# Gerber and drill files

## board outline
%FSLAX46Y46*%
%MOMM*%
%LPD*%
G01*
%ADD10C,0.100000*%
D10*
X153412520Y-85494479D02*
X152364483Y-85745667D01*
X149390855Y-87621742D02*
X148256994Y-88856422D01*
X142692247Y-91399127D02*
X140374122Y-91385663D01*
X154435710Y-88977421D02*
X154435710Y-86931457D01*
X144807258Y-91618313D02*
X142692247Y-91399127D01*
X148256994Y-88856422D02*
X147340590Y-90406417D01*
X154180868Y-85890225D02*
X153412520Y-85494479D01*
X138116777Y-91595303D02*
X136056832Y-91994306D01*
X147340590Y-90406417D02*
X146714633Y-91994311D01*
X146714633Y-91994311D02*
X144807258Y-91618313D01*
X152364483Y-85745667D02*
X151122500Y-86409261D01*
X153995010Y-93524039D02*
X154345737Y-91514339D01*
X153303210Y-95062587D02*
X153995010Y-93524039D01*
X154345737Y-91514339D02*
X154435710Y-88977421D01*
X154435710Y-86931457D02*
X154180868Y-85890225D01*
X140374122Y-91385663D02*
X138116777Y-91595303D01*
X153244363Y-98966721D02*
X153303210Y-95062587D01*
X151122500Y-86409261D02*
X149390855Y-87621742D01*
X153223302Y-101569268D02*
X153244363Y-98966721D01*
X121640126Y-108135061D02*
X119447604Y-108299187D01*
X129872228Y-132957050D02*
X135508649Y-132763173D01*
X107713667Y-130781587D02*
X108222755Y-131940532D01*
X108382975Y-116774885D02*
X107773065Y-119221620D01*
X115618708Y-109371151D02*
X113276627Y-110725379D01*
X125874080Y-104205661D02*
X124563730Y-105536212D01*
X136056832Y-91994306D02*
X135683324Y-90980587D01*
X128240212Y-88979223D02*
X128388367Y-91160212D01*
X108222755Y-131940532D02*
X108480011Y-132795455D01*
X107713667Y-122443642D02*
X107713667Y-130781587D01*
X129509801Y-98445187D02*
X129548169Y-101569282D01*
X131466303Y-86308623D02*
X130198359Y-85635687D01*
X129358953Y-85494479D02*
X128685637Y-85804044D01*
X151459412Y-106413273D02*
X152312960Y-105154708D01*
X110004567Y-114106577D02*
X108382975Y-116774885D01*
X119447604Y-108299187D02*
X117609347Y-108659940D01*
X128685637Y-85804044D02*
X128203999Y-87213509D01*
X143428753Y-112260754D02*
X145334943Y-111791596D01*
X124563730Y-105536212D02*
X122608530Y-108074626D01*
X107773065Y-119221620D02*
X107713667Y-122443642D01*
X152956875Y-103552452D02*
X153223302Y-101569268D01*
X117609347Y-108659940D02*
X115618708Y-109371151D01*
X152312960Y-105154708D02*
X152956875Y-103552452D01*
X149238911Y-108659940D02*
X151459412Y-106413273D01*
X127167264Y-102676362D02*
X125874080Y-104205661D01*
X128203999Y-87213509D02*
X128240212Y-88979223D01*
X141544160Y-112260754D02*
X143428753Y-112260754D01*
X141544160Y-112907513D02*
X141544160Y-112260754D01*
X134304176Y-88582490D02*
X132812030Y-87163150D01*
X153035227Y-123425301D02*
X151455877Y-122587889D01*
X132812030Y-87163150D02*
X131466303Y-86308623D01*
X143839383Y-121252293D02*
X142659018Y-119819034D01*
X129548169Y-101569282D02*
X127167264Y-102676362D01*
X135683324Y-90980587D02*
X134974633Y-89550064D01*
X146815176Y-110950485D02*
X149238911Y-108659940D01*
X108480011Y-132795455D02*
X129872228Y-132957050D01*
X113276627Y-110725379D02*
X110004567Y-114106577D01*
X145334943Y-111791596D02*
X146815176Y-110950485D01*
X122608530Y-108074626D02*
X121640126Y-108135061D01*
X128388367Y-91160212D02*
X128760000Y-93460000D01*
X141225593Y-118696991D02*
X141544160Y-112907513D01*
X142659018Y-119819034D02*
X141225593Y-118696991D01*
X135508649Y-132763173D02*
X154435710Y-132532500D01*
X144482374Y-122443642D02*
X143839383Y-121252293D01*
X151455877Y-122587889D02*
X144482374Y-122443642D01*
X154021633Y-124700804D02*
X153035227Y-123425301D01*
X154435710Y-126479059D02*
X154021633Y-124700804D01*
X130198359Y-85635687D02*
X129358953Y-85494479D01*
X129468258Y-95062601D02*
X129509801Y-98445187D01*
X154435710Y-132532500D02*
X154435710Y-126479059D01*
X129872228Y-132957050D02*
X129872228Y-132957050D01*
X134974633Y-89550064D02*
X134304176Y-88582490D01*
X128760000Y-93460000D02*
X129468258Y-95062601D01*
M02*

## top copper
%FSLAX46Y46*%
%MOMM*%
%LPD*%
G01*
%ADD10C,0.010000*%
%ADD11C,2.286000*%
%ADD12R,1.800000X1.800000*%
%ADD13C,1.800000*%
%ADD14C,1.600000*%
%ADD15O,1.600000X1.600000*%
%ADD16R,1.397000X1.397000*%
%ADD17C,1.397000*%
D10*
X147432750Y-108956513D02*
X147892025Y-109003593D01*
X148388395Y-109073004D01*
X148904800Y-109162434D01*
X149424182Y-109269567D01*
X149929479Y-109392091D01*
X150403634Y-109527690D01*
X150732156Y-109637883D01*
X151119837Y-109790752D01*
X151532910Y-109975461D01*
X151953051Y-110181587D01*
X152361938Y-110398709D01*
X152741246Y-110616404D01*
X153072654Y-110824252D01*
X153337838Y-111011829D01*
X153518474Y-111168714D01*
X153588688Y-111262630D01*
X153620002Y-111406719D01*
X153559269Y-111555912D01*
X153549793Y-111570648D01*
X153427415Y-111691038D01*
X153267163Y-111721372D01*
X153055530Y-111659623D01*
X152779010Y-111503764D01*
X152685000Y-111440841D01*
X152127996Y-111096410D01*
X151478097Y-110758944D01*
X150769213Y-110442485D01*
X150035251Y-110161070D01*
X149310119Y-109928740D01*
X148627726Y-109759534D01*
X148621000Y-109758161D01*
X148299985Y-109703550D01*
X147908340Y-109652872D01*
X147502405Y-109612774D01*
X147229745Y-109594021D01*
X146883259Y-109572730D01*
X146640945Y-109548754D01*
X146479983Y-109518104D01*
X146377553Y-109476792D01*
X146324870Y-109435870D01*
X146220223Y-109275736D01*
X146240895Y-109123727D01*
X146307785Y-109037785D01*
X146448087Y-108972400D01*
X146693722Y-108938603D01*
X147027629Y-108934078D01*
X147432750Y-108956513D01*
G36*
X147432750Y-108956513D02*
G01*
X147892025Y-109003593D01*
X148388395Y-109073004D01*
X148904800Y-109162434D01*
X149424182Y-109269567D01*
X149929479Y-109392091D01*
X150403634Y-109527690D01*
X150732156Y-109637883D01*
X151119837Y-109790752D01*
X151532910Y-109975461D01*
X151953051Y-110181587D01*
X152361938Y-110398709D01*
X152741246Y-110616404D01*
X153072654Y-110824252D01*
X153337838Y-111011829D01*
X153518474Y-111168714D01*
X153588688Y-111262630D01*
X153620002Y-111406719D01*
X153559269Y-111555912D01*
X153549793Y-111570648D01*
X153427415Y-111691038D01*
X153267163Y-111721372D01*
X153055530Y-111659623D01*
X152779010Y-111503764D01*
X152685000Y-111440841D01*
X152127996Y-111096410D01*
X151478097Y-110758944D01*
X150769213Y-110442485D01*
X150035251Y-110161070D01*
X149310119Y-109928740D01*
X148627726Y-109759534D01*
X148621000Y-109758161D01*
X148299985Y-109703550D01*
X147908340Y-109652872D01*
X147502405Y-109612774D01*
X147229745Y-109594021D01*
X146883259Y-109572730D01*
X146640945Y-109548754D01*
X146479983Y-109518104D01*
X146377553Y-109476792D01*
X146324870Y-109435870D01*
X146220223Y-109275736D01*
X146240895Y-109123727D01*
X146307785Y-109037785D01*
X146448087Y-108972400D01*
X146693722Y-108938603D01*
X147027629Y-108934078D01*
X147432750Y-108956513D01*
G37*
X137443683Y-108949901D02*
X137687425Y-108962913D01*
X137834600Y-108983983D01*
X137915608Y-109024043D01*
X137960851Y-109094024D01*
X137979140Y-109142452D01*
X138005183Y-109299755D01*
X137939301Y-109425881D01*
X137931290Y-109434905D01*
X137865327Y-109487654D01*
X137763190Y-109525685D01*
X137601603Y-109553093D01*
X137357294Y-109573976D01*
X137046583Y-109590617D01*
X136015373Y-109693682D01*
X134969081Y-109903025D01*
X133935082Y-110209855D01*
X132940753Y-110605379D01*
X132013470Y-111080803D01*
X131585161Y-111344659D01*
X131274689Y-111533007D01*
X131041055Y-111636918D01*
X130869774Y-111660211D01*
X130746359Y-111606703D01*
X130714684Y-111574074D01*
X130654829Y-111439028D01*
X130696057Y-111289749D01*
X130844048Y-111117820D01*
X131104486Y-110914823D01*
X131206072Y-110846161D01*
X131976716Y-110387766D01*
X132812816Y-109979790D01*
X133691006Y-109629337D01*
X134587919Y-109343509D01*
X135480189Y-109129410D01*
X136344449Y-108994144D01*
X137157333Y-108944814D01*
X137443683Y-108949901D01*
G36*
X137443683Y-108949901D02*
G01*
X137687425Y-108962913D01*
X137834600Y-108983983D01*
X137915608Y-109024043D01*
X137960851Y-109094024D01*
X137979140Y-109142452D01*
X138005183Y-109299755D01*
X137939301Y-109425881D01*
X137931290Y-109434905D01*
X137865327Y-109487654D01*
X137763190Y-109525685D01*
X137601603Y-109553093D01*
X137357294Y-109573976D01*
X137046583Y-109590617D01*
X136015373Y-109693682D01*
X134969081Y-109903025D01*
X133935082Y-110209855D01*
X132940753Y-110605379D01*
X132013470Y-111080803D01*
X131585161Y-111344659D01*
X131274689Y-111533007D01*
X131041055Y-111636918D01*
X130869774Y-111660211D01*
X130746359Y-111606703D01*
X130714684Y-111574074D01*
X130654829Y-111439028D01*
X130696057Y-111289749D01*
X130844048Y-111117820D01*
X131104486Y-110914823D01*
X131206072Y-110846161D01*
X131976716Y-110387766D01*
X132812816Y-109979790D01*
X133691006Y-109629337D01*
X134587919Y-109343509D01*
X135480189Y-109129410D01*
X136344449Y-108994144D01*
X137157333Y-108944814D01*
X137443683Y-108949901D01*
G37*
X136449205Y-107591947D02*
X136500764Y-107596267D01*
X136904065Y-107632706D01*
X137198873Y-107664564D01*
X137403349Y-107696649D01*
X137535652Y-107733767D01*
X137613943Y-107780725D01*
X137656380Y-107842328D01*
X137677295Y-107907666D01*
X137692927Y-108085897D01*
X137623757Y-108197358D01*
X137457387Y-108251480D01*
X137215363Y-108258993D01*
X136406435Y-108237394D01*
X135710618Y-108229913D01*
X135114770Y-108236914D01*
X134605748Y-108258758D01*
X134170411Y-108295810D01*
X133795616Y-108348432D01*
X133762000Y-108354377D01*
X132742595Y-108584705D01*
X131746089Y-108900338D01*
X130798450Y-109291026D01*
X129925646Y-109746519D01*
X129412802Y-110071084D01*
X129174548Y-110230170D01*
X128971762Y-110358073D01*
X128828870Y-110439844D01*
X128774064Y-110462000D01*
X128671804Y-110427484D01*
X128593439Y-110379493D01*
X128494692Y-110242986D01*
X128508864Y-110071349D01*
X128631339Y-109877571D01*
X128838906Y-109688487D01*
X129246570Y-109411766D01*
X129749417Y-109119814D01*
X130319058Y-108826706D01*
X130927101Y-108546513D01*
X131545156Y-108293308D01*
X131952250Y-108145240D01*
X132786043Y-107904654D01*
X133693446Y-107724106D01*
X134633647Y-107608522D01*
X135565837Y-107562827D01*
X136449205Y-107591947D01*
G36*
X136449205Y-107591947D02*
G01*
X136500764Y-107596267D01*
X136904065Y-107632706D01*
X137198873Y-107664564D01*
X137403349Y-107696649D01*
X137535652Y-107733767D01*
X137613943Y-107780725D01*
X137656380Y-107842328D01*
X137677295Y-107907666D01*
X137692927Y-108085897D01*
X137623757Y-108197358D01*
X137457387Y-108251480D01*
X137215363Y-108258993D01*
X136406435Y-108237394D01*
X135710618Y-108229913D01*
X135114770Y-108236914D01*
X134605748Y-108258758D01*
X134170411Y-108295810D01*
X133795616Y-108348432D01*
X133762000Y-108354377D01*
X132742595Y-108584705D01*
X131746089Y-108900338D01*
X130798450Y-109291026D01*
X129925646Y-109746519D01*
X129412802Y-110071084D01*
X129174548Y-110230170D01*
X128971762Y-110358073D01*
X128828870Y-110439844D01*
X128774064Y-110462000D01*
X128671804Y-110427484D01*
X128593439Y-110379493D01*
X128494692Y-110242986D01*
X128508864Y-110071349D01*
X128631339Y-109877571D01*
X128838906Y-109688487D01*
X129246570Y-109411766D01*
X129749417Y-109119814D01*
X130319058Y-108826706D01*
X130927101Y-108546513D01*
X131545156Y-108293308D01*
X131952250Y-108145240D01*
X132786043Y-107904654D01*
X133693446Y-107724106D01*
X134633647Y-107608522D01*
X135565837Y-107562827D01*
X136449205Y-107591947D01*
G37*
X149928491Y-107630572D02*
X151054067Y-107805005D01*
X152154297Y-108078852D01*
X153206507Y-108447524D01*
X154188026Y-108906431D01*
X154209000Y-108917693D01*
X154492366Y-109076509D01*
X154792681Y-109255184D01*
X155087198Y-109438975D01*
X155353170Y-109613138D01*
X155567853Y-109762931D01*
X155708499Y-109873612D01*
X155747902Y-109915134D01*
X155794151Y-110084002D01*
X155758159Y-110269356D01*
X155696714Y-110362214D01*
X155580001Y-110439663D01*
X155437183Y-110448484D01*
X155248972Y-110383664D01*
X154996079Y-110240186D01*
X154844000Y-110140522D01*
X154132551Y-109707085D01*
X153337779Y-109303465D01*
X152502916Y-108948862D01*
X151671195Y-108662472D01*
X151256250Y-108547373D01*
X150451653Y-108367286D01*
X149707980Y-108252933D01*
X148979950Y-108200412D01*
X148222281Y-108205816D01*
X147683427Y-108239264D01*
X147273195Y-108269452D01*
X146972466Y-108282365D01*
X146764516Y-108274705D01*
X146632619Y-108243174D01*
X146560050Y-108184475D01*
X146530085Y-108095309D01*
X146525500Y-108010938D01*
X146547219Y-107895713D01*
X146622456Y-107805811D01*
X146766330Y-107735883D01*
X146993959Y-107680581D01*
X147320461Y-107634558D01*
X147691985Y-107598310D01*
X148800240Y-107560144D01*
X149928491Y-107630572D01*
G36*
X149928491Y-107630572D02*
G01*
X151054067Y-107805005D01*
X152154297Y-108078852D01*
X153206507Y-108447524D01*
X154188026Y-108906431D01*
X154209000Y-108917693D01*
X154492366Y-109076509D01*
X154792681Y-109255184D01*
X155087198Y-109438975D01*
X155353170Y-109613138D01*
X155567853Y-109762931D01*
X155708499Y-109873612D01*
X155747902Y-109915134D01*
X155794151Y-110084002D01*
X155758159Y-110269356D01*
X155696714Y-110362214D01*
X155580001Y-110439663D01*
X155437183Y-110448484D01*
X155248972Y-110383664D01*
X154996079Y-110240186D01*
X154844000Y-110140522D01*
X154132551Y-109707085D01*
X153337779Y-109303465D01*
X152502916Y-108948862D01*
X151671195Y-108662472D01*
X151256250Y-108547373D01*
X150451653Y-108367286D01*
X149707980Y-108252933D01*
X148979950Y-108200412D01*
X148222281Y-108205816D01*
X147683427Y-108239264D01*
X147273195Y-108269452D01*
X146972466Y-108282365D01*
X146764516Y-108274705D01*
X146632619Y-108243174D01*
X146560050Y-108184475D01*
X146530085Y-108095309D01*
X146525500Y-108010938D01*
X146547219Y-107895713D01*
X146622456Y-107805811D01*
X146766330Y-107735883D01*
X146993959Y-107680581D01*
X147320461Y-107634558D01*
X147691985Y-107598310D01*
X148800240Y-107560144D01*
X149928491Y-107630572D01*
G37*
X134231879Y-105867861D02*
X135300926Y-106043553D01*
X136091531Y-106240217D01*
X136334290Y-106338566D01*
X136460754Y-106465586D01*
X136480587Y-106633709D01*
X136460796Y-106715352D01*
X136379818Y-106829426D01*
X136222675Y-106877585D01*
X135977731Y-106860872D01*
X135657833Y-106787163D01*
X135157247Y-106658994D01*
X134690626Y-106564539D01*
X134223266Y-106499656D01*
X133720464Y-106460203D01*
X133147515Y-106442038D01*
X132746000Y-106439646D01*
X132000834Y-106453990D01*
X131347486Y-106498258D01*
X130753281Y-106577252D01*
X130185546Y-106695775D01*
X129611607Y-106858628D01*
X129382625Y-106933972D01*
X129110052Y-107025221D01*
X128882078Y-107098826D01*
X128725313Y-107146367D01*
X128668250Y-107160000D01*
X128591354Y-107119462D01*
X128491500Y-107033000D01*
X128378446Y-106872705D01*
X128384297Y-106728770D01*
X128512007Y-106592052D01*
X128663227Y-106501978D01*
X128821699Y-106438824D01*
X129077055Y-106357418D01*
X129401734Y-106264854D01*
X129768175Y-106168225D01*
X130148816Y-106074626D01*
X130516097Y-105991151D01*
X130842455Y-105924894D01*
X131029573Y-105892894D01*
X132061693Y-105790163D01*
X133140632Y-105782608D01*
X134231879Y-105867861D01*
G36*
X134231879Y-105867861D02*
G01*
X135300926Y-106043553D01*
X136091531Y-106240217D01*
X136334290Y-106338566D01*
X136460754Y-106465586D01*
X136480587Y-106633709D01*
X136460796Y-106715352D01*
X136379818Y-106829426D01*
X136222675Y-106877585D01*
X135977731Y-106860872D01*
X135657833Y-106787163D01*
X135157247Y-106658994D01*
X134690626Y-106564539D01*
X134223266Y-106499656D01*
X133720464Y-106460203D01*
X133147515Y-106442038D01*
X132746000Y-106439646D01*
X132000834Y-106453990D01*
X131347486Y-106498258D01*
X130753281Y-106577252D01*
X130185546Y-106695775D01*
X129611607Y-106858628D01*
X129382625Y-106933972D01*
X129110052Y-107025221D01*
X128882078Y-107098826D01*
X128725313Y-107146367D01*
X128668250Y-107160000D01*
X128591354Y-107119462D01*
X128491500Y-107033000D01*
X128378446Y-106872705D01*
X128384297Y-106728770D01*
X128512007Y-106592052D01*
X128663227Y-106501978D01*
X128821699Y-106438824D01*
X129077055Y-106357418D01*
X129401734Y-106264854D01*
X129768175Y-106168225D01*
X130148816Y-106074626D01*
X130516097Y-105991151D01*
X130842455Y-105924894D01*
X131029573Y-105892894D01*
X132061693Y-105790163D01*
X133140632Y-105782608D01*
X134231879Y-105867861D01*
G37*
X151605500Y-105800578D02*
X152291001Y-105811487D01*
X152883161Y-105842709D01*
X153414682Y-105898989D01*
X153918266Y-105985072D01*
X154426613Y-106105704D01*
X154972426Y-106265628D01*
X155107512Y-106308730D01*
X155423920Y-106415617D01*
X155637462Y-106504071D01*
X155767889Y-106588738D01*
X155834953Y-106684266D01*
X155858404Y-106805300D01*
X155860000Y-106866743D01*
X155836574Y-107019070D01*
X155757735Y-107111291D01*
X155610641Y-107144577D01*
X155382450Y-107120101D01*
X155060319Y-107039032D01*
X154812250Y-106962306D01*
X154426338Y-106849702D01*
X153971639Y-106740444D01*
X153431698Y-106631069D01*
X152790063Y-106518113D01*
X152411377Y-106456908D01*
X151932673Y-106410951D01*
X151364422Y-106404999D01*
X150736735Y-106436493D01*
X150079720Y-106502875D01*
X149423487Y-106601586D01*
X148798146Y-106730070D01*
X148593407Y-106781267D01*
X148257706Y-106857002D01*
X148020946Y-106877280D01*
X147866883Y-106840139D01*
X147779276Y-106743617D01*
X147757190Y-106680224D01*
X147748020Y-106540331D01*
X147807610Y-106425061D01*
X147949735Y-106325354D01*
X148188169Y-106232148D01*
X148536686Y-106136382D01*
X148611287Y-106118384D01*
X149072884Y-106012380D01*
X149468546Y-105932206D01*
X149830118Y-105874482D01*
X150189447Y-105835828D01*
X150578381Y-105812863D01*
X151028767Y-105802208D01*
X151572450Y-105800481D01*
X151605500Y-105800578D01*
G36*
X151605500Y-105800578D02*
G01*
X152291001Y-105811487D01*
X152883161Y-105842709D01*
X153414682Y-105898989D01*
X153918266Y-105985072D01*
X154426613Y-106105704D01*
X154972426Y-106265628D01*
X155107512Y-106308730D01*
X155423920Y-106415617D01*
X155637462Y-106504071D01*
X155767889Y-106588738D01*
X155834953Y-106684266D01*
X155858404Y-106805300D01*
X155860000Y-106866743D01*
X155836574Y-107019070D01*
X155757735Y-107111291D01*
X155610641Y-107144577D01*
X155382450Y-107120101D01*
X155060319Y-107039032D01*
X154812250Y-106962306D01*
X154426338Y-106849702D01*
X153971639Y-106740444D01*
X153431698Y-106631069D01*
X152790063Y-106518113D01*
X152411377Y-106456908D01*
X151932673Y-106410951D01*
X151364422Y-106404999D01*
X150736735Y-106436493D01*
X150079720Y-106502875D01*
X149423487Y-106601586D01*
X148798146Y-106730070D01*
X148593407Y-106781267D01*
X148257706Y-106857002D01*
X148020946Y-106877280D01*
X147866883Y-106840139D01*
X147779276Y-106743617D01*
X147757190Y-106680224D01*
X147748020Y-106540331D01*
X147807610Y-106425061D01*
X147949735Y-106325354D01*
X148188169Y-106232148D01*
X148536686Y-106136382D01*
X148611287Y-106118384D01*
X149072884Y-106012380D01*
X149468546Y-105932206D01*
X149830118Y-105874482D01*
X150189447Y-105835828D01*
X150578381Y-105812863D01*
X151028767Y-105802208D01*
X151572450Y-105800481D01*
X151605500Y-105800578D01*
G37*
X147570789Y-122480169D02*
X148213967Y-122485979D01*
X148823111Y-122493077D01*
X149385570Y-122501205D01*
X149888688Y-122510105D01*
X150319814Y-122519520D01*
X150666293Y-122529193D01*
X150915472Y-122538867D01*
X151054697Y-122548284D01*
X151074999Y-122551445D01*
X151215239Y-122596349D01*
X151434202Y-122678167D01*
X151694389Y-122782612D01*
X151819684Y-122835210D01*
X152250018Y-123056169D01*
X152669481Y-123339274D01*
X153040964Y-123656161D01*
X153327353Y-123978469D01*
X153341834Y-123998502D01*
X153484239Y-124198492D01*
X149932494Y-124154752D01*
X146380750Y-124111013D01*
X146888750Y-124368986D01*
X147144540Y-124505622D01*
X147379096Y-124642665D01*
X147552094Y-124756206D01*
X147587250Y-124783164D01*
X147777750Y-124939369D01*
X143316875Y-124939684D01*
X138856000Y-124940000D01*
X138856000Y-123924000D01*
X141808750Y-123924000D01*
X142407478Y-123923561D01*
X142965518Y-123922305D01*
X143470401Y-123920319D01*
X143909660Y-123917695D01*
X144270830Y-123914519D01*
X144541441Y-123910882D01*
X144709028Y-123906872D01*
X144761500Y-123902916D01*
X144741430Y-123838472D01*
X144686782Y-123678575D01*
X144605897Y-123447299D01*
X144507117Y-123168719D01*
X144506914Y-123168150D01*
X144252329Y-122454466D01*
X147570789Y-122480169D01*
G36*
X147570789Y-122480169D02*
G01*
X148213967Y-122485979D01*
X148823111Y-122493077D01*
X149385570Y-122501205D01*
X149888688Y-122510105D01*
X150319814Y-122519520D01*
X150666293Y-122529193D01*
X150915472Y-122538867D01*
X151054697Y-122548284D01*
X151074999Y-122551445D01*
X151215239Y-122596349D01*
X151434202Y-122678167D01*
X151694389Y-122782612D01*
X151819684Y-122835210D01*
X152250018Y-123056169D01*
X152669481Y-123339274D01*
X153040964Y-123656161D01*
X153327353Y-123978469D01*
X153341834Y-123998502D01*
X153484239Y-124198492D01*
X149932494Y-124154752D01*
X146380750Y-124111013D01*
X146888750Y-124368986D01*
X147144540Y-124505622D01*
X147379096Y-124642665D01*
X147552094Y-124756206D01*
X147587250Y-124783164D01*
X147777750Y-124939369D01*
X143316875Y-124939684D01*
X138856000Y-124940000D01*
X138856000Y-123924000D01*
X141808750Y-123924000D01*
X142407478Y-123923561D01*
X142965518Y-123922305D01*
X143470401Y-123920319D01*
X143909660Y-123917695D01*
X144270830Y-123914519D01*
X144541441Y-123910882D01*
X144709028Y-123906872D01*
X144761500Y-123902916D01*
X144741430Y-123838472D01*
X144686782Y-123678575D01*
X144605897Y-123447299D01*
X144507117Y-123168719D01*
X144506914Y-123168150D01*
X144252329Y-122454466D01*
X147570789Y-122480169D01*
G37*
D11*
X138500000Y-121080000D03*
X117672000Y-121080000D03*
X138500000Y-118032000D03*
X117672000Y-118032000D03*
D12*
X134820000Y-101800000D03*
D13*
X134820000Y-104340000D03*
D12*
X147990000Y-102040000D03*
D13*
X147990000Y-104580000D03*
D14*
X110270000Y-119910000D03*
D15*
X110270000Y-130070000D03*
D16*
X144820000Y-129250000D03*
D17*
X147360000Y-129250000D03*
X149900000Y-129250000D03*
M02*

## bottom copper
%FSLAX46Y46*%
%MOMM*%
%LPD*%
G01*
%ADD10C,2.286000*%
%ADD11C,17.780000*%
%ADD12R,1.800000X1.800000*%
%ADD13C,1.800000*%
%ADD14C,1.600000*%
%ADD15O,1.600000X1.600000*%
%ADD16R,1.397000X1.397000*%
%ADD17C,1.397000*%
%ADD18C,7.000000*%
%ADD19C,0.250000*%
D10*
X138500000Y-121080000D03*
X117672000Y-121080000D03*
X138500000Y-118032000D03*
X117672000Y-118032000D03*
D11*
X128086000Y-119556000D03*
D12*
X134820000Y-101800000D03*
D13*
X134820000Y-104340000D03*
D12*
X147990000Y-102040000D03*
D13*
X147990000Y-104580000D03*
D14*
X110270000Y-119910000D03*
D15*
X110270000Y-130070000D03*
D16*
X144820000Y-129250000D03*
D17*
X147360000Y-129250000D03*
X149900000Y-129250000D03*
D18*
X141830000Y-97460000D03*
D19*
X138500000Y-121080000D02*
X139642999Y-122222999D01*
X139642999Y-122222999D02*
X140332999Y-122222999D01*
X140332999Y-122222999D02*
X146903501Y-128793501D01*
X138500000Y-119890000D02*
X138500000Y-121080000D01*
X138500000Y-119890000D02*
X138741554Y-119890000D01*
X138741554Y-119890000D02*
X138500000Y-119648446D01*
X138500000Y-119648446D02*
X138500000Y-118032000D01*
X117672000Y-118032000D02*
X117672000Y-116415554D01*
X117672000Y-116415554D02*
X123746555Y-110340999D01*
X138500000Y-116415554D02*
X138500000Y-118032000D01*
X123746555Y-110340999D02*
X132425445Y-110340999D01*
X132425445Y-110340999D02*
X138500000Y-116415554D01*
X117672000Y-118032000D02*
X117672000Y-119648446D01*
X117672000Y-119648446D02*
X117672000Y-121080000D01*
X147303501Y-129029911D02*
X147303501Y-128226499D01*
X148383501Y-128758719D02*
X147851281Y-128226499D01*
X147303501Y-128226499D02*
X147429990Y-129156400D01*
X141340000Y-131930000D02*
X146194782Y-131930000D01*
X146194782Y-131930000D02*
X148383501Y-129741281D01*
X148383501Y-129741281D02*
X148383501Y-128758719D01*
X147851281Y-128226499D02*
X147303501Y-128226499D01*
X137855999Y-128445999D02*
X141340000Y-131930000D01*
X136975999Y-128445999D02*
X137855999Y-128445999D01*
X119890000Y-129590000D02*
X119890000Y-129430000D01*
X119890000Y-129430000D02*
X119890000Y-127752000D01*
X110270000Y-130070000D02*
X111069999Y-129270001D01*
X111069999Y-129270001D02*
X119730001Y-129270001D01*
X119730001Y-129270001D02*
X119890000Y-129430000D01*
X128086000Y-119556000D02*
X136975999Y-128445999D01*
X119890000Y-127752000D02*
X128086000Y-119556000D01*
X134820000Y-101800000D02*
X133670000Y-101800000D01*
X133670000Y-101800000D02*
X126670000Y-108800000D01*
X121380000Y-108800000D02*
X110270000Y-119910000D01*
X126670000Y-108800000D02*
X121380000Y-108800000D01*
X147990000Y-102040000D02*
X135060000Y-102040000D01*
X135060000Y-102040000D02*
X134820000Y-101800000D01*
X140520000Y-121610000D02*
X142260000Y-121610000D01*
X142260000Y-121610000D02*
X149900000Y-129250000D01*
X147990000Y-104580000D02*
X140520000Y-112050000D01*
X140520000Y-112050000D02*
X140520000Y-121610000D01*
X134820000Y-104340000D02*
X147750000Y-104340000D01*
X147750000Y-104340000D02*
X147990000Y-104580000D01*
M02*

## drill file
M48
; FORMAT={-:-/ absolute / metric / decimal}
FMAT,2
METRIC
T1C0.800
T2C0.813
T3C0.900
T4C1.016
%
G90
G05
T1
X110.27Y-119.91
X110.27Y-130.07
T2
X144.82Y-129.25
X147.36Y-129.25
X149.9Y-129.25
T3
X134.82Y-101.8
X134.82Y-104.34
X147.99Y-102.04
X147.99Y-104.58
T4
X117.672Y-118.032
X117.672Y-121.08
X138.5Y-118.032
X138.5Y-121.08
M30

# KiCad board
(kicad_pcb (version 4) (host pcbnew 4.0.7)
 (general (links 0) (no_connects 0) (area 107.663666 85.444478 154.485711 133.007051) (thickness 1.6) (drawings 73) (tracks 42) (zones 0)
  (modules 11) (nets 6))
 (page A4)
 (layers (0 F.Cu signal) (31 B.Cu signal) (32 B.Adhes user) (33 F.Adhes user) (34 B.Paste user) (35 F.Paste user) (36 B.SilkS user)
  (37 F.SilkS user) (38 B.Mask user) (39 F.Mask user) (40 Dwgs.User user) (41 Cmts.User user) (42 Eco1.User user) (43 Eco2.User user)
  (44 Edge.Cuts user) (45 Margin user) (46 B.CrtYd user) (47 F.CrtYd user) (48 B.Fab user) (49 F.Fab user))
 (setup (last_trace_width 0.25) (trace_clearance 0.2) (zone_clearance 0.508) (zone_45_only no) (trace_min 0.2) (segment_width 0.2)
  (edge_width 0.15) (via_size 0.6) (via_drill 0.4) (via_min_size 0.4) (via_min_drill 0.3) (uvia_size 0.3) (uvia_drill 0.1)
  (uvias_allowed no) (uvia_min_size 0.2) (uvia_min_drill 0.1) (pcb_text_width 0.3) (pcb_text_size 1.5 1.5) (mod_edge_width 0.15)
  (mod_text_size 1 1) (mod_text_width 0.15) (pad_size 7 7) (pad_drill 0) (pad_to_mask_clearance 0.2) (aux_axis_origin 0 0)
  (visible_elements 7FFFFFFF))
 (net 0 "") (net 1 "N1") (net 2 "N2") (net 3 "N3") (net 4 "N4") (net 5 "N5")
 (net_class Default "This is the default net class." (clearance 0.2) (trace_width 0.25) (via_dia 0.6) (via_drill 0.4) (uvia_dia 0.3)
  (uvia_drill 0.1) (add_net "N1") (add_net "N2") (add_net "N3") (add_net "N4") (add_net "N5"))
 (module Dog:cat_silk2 (layer F.Cu) (at 130.76 109.63)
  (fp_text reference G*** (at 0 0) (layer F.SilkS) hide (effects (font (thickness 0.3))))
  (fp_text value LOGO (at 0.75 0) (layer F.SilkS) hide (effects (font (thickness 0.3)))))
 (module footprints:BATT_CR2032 (layer B.Cu) (at 128.086 119.556 180)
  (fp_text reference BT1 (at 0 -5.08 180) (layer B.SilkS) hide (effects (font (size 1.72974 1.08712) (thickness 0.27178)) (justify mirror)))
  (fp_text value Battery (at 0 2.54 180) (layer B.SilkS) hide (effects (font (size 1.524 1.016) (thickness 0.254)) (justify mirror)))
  (pad 1 thru_hole circle (at -10.414 -1.524 180) (size 2.286 2.286) (drill 1.016) (layers *.Cu *.Mask B.SilkS) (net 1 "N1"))
  (pad 1 thru_hole circle (at 10.414 -1.524 180) (size 2.286 2.286) (drill 1.016) (layers *.Cu *.Mask B.SilkS) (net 1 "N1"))
  (pad 1 thru_hole circle (at -10.414 1.524 180) (size 2.286 2.286) (drill 1.016) (layers *.Cu *.Mask B.SilkS) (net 1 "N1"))
  (pad 1 thru_hole circle (at 10.414 1.524 180) (size 2.286 2.286) (drill 1.016) (layers *.Cu *.Mask B.SilkS) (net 1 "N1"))
  (pad 2 smd circle (at 0 0 180) (size 17.78 17.78) (layers B.Cu B.Paste B.Mask) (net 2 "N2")))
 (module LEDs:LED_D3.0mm (layer F.Cu) (at 134.82 101.8 270)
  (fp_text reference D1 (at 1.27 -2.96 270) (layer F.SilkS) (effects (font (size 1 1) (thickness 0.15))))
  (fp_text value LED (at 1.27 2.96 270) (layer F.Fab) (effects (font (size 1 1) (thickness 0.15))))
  (pad 1 thru_hole rect (at 0 0 270) (size 1.8 1.8) (drill 0.9) (layers *.Cu *.Mask) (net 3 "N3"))
  (pad 2 thru_hole circle (at 2.54 0 270) (size 1.8 1.8) (drill 0.9) (layers *.Cu *.Mask) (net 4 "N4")))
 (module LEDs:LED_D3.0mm (layer F.Cu) (at 147.99 102.04 270)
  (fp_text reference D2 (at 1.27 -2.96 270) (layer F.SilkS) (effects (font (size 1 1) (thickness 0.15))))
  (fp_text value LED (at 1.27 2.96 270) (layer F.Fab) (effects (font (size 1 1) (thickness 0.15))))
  (pad 1 thru_hole rect (at 0 0 270) (size 1.8 1.8) (drill 0.9) (layers *.Cu *.Mask) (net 3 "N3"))
  (pad 2 thru_hole circle (at 2.54 0 270) (size 1.8 1.8) (drill 0.9) (layers *.Cu *.Mask) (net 4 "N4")))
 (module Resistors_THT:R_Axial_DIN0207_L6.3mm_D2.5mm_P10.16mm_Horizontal (layer B.Cu) (at 110.27 119.91 270)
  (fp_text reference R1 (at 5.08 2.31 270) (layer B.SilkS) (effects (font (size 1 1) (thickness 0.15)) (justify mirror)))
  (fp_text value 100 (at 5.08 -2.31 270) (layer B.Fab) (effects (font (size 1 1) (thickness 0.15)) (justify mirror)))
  (pad 1 thru_hole circle (at 0 0 270) (size 1.6 1.6) (drill 0.8) (layers *.Cu *.Mask) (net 3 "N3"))
  (pad 2 thru_hole oval (at 10.16 0 270) (size 1.6 1.6) (drill 0.8) (layers *.Cu *.Mask) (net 2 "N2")))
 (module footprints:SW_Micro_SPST (layer B.Cu) (at 147.36 129.25)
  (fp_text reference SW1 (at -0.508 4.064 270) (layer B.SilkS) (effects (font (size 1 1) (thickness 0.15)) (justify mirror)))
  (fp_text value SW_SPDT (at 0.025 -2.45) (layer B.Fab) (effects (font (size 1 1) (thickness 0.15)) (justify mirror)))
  (pad 1 thru_hole rect (at -2.54 0) (size 1.397 1.397) (drill 0.8128) (layers *.Cu *.Mask B.SilkS) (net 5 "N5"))
  (pad 2 thru_hole circle (at 0 0) (size 1.397 1.397) (drill 0.8128) (layers *.Cu *.Mask B.SilkS) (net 1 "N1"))
  (pad 3 thru_hole circle (at 2.54 0) (size 1.397 1.397) (drill 0.8128) (layers *.Cu *.Mask B.SilkS) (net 4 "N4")))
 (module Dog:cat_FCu (layer F.Cu) (at 131.73 110.97)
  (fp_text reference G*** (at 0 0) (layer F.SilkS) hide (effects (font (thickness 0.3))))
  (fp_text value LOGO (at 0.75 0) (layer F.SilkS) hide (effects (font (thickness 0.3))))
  (fp_poly
   (pts (xy 15.70275 -2.013487) (xy 16.162025 -1.966407) (xy 16.658395 -1.896996) (xy 17.1748 -1.807566) (xy 17.694182 -1.700433)
    (xy 18.199479 -1.577909) (xy 18.673634 -1.44231) (xy 19.002156 -1.332117) (xy 19.389837 -1.179248) (xy 19.80291 -0.994539)
    (xy 20.223051 -0.788413) (xy 20.631938 -0.571291) (xy 21.011246 -0.353596) (xy 21.342654 -0.145748) (xy 21.607838 0.041829)
    (xy 21.788474 0.198714) (xy 21.858688 0.29263) (xy 21.890002 0.436719) (xy 21.829269 0.585912) (xy 21.819793 0.600648)
    (xy 21.697415 0.721038) (xy 21.537163 0.751372) (xy 21.32553 0.689623) (xy 21.04901 0.533764) (xy 20.955 0.470841)
    (xy 20.397996 0.12641) (xy 19.748097 -0.211056) (xy 19.039213 -0.527515) (xy 18.305251 -0.80893) (xy 17.580119 -1.04126)
    (xy 16.897726 -1.210466) (xy 16.891 -1.211839) (xy 16.569985 -1.26645) (xy 16.17834 -1.317128) (xy 15.772405 -1.357226)
    (xy 15.499745 -1.375979) (xy 15.153259 -1.39727) (xy 14.910945 -1.421246) (xy 14.749983 -1.451896) (xy 14.647553 -1.493208)
    (xy 14.59487 -1.53413) (xy 14.490223 -1.694264) (xy 14.510895 -1.846273) (xy 14.577785 -1.932215) (xy 14.718087 -1.9976)
    (xy 14.963722 -2.031397) (xy 15.297629 -2.035922) (xy 15.70275 -2.013487))
   (layer F.Cu) (width 0.01))
  (fp_poly
   (pts (xy 5.713683 -2.020099) (xy 5.957425 -2.007087) (xy 6.1046 -1.986017) (xy 6.185608 -1.945957) (xy 6.230851 -1.875976)
    (xy 6.24914 -1.827548) (xy 6.275183 -1.670245) (xy 6.209301 -1.544119) (xy 6.20129 -1.535095) (xy 6.135327 -1.482346)
    (xy 6.03319 -1.444315) (xy 5.871603 -1.416907) (xy 5.627294 -1.396024) (xy 5.316583 -1.379383) (xy 4.285373 -1.276318)
    (xy 3.239081 -1.066975) (xy 2.205082 -0.760145) (xy 1.210753 -0.364621) (xy 0.28347 0.110803) (xy -0.144839 0.374659)
    (xy -0.455311 0.563007) (xy -0.688945 0.666918) (xy -0.860226 0.690211) (xy -0.983641 0.636703) (xy -1.015316 0.604074)
    (xy -1.075171 0.469028) (xy -1.033943 0.319749) (xy -0.885952 0.14782) (xy -0.625514 -0.055177) (xy -0.523928 -0.123839)
    (xy 0.246716 -0.582234) (xy 1.082816 -0.99021) (xy 1.961006 -1.340663) (xy 2.857919 -1.626491) (xy 3.750189 -1.84059)
    (xy 4.614449 -1.975856) (xy 5.427333 -2.025186) (xy 5.713683 -2.020099))
   (layer F.Cu) (width 0.01))
  (fp_poly
   (pts (xy 4.719205 -3.378053) (xy 4.770764 -3.373733) (xy 5.174065 -3.337294) (xy 5.468873 -3.305436) (xy 5.673349 -3.273351)
    (xy 5.805652 -3.236233) (xy 5.883943 -3.189275) (xy 5.92638 -3.127672) (xy 5.947295 -3.062334) (xy 5.962927 -2.884103)
    (xy 5.893757 -2.772642) (xy 5.727387 -2.71852) (xy 5.485363 -2.711007) (xy 4.676435 -2.732606) (xy 3.980618 -2.740087)
    (xy 3.38477 -2.733086) (xy 2.875748 -2.711242) (xy 2.440411 -2.67419) (xy 2.065616 -2.621568) (xy 2.032 -2.615623)
    (xy 1.012595 -2.385295) (xy 0.016089 -2.069662) (xy -0.93155 -1.678974) (xy -1.804354 -1.223481) (xy -2.317198 -0.898916)
    (xy -2.555452 -0.73983) (xy -2.758238 -0.611927) (xy -2.90113 -0.530156) (xy -2.955936 -0.508) (xy -3.058196 -0.542516)
    (xy -3.136561 -0.590507) (xy -3.235308 -0.727014) (xy -3.221136 -0.898651) (xy -3.098661 -1.092429) (xy -2.891094 -1.281513)
    (xy -2.48343 -1.558234) (xy -1.980583 -1.850186) (xy -1.410942 -2.143294) (xy -0.802899 -2.423487) (xy -0.184844 -2.676692)
    (xy 0.22225 -2.82476) (xy 1.056043 -3.065346) (xy 1.963446 -3.245894) (xy 2.903647 -3.361478) (xy 3.835837 -3.407173)
    (xy 4.719205 -3.378053))
   (layer F.Cu) (width 0.01))
  (fp_poly
   (pts (xy 18.198491 -3.339428) (xy 19.324067 -3.164995) (xy 20.424297 -2.891148) (xy 21.476507 -2.522476) (xy 22.458026 -2.063569)
    (xy 22.479 -2.052307) (xy 22.762366 -1.893491) (xy 23.062681 -1.714816) (xy 23.357198 -1.531025) (xy 23.62317 -1.356862)
    (xy 23.837853 -1.207069) (xy 23.978499 -1.096388) (xy 24.017902 -1.054866) (xy 24.064151 -0.885998) (xy 24.028159 -0.700644)
    (xy 23.966714 -0.607786) (xy 23.850001 -0.530337) (xy 23.707183 -0.521516) (xy 23.518972 -0.586336) (xy 23.266079 -0.729814)
    (xy 23.114 -0.829478) (xy 22.402551 -1.262915) (xy 21.607779 -1.666535) (xy 20.772916 -2.021138) (xy 19.941195 -2.307528)
    (xy 19.52625 -2.422627) (xy 18.721653 -2.602714) (xy 17.97798 -2.717067) (xy 17.24995 -2.769588) (xy 16.492281 -2.764184)
    (xy 15.953427 -2.730736) (xy 15.543195 -2.700548) (xy 15.242466 -2.687635) (xy 15.034516 -2.695295) (xy 14.902619 -2.726826)
    (xy 14.83005 -2.785525) (xy 14.800085 -2.874691) (xy 14.7955 -2.959062) (xy 14.817219 -3.074287) (xy 14.892456 -3.164189)
    (xy 15.03633 -3.234117) (xy 15.263959 -3.289419) (xy 15.590461 -3.335442) (xy 15.961985 -3.37169) (xy 17.07024 -3.409856)
    (xy 18.198491 -3.339428))
   (layer F.Cu) (width 0.01))
  (fp_poly
   (pts (xy 2.501879 -5.102139) (xy 3.570926 -4.926447) (xy 4.361531 -4.729783) (xy 4.60429 -4.631434) (xy 4.730754 -4.504414)
    (xy 4.750587 -4.336291) (xy 4.730796 -4.254648) (xy 4.649818 -4.140574) (xy 4.492675 -4.092415) (xy 4.247731 -4.109128)
    (xy 3.927833 -4.182837) (xy 3.427247 -4.311006) (xy 2.960626 -4.405461) (xy 2.493266 -4.470344) (xy 1.990464 -4.509797)
    (xy 1.417515 -4.527962) (xy 1.016 -4.530354) (xy 0.270834 -4.51601) (xy -0.382514 -4.471742) (xy -0.976719 -4.392748)
    (xy -1.544454 -4.274225) (xy -2.118393 -4.111372) (xy -2.347375 -4.036028) (xy -2.619948 -3.944779) (xy -2.847922 -3.871174)
    (xy -3.004687 -3.823633) (xy -3.06175 -3.81) (xy -3.138646 -3.850538) (xy -3.2385 -3.937) (xy -3.351554 -4.097295)
    (xy -3.345703 -4.24123) (xy -3.217993 -4.377948) (xy -3.066773 -4.468022) (xy -2.908301 -4.531176) (xy -2.652945 -4.612582)
    (xy -2.328266 -4.705146) (xy -1.961825 -4.801775) (xy -1.581184 -4.895374) (xy -1.213903 -4.978849) (xy -0.887545 -5.045106)
    (xy -0.700427 -5.077106) (xy 0.331693 -5.179837) (xy 1.410632 -5.187392) (xy 2.501879 -5.102139))
   (layer F.Cu) (width 0.01))
  (fp_poly
   (pts (xy 19.8755 -5.169422) (xy 20.561001 -5.158513) (xy 21.153161 -5.127291) (xy 21.684682 -5.071011) (xy 22.188266 -4.984928)
    (xy 22.696613 -4.864296) (xy 23.242426 -4.704372) (xy 23.377512 -4.66127) (xy 23.69392 -4.554383) (xy 23.907462 -4.465929)
    (xy 24.037889 -4.381262) (xy 24.104953 -4.285734) (xy 24.128404 -4.1647) (xy 24.13 -4.103257) (xy 24.106574 -3.95093)
    (xy 24.027735 -3.858709) (xy 23.880641 -3.825423) (xy 23.65245 -3.849899) (xy 23.330319 -3.930968) (xy 23.08225 -4.007694)
    (xy 22.696338 -4.120298) (xy 22.241639 -4.229556) (xy 21.701698 -4.338931) (xy 21.060063 -4.451887) (xy 20.681377 -4.513092)
    (xy 20.202673 -4.559049) (xy 19.634422 -4.565001) (xy 19.006735 -4.533507) (xy 18.34972 -4.467125) (xy 17.693487 -4.368414)
    (xy 17.068146 -4.23993) (xy 16.863407 -4.188733) (xy 16.527706 -4.112998) (xy 16.290946 -4.09272) (xy 16.136883 -4.129861)
    (xy 16.049276 -4.226383) (xy 16.02719 -4.289776) (xy 16.01802 -4.429669) (xy 16.07761 -4.544939) (xy 16.219735 -4.644646)
    (xy 16.458169 -4.737852) (xy 16.806686 -4.833618) (xy 16.881287 -4.851616) (xy 17.342884 -4.95762) (xy 17.738546 -5.037794)
    (xy 18.100118 -5.095518) (xy 18.459447 -5.134172) (xy 18.848381 -5.157137) (xy 19.298767 -5.167792) (xy 19.84245 -5.169519)
    (xy 19.8755 -5.169422))
   (layer F.Cu) (width 0.01)))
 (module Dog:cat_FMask (layer F.Cu) (at 131.7 111)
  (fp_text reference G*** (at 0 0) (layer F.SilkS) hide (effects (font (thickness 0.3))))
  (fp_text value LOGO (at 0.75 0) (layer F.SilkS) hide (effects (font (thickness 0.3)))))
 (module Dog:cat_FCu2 (layer F.Cu) (at 131.49 109.7)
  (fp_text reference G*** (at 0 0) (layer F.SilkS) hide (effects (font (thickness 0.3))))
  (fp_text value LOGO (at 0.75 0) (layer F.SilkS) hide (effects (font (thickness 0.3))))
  (fp_poly
   (pts (xy 16.080789 12.780169) (xy 16.723967 12.785979) (xy 17.333111 12.793077) (xy 17.89557 12.801205) (xy 18.398688 12.810105)
    (xy 18.829814 12.81952) (xy 19.176293 12.829193) (xy 19.425472 12.838867) (xy 19.564697 12.848284) (xy 19.584999 12.851445)
    (xy 19.725239 12.896349) (xy 19.944202 12.978167) (xy 20.204389 13.082612) (xy 20.329684 13.13521) (xy 20.760018 13.356169)
    (xy 21.179481 13.639274) (xy 21.550964 13.956161) (xy 21.837353 14.278469) (xy 21.851834 14.298502) (xy 21.994239 14.498492)
    (xy 18.442494 14.454752) (xy 14.89075 14.411013) (xy 15.39875 14.668986) (xy 15.65454 14.805622) (xy 15.889096 14.942665)
    (xy 16.062094 15.056206) (xy 16.09725 15.083164) (xy 16.28775 15.239369) (xy 11.826875 15.239684) (xy 7.366 15.24) (xy 7.366 14.224)
    (xy 10.31875 14.224) (xy 10.917478 14.223561) (xy 11.475518 14.222305) (xy 11.980401 14.220319) (xy 12.41966 14.217695)
    (xy 12.78083 14.214519) (xy 13.051441 14.210882) (xy 13.219028 14.206872) (xy 13.2715 14.202916) (xy 13.25143 14.138472)
    (xy 13.196782 13.978575) (xy 13.115897 13.747299) (xy 13.017117 13.468719) (xy 13.016914 13.46815) (xy 12.762329 12.754466)
    (xy 16.080789 12.780169))
   (layer F.Cu) (width 0.01)))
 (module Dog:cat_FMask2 (layer F.Cu) (at 131.37 109.67)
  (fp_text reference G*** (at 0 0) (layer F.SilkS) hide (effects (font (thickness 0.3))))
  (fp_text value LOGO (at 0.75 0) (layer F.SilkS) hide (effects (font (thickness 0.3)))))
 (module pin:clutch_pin (layer F.Cu) (at 141.83 97.46)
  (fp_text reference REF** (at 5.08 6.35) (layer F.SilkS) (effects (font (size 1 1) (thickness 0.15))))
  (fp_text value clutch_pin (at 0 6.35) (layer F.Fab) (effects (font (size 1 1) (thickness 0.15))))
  (pad 1 smd circle (at 0 0 90) (size 7 7) (layers B.Cu B.Paste B.SilkS B.Mask)))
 (gr_line (start 153.41252 85.494479) (end 152.364483 85.745667) (layer Edge.Cuts) (width 0.1))
 (gr_line (start 149.390855 87.621742) (end 148.256994 88.856422) (layer Edge.Cuts) (width 0.1))
 (gr_line (start 142.692247 91.399127) (end 140.374122 91.385663) (layer Edge.Cuts) (width 0.1))
 (gr_line (start 154.43571 88.977421) (end 154.43571 86.931457) (layer Edge.Cuts) (width 0.1))
 (gr_line (start 144.807258 91.618313) (end 142.692247 91.399127) (layer Edge.Cuts) (width 0.1))
 (gr_line (start 148.256994 88.856422) (end 147.34059 90.406417) (layer Edge.Cuts) (width 0.1))
 (gr_line (start 154.180868 85.890225) (end 153.41252 85.494479) (layer Edge.Cuts) (width 0.1))
 (gr_line (start 138.116777 91.595303) (end 136.056832 91.994306) (layer Edge.Cuts) (width 0.1))
 (gr_line (start 147.34059 90.406417) (end 146.714633 91.994311) (layer Edge.Cuts) (width 0.1))
 (gr_line (start 146.714633 91.994311) (end 144.807258 91.618313) (layer Edge.Cuts) (width 0.1))
 (gr_line (start 152.364483 85.745667) (end 151.1225 86.409261) (layer Edge.Cuts) (width 0.1))
 (gr_line (start 153.99501 93.524039) (end 154.345737 91.514339) (layer Edge.Cuts) (width 0.1))
 (gr_line (start 153.30321 95.062587) (end 153.99501 93.524039) (layer Edge.Cuts) (width 0.1))
 (gr_line (start 154.345737 91.514339) (end 154.43571 88.977421) (layer Edge.Cuts) (width 0.1))
 (gr_line (start 154.43571 86.931457) (end 154.180868 85.890225) (layer Edge.Cuts) (width 0.1))
 (gr_line (start 140.374122 91.385663) (end 138.116777 91.595303) (layer Edge.Cuts) (width 0.1))
 (gr_line (start 153.244363 98.966721) (end 153.30321 95.062587) (layer Edge.Cuts) (width 0.1))
 (gr_line (start 151.1225 86.409261) (end 149.390855 87.621742) (layer Edge.Cuts) (width 0.1))
 (gr_line (start 153.223302 101.569268) (end 153.244363 98.966721) (layer Edge.Cuts) (width 0.1))
 (gr_line (start 121.640126 108.135061) (end 119.447604 108.299187) (layer Edge.Cuts) (width 0.1))
 (gr_line (start 129.872228 132.95705) (end 135.508649 132.763173) (layer Edge.Cuts) (width 0.1))
 (gr_line (start 107.713667 130.781587) (end 108.222755 131.940532) (layer Edge.Cuts) (width 0.1))
 (gr_line (start 108.382975 116.774885) (end 107.773065 119.22162) (layer Edge.Cuts) (width 0.1))
 (gr_line (start 115.618708 109.371151) (end 113.276627 110.725379) (layer Edge.Cuts) (width 0.1))
 (gr_line (start 125.87408 104.205661) (end 124.56373 105.536212) (layer Edge.Cuts) (width 0.1))
 (gr_line (start 136.056832 91.994306) (end 135.683324 90.980587) (layer Edge.Cuts) (width 0.1))
 (gr_line (start 128.240212 88.979223) (end 128.388367 91.160212) (layer Edge.Cuts) (width 0.1))
 (gr_line (start 108.222755 131.940532) (end 108.480011 132.795455) (layer Edge.Cuts) (width 0.1))
 (gr_line (start 107.713667 122.443642) (end 107.713667 130.781587) (layer Edge.Cuts) (width 0.1))
 (gr_line (start 129.509801 98.445187) (end 129.548169 101.569282) (layer Edge.Cuts) (width 0.1))
 (gr_line (start 131.466303 86.308623) (end 130.198359 85.635687) (layer Edge.Cuts) (width 0.1))
 (gr_line (start 129.358953 85.494479) (end 128.685637 85.804044) (layer Edge.Cuts) (width 0.1))
 (gr_line (start 151.459412 106.413273) (end 152.31296 105.154708) (layer Edge.Cuts) (width 0.1))
 (gr_line (start 110.004567 114.106577) (end 108.382975 116.774885) (layer Edge.Cuts) (width 0.1))
 (gr_line (start 119.447604 108.299187) (end 117.609347 108.65994) (layer Edge.Cuts) (width 0.1))
 (gr_line (start 128.685637 85.804044) (end 128.203999 87.213509) (layer Edge.Cuts) (width 0.1))
 (gr_line (start 143.428753 112.260754) (end 145.334943 111.791596) (layer Edge.Cuts) (width 0.1))
 (gr_line (start 124.56373 105.536212) (end 122.60853 108.074626) (layer Edge.Cuts) (width 0.1))
 (gr_line (start 107.773065 119.22162) (end 107.713667 122.443642) (layer Edge.Cuts) (width 0.1))
 (gr_line (start 152.956875 103.552452) (end 153.223302 101.569268) (layer Edge.Cuts) (width 0.1))
 (gr_line (start 117.609347 108.65994) (end 115.618708 109.371151) (layer Edge.Cuts) (width 0.1))
 (gr_line (start 152.31296 105.154708) (end 152.956875 103.552452) (layer Edge.Cuts) (width 0.1))
 (gr_line (start 149.238911 108.65994) (end 151.459412 106.413273) (layer Edge.Cuts) (width 0.1))
 (gr_line (start 127.167264 102.676362) (end 125.87408 104.205661) (layer Edge.Cuts) (width 0.1))
 (gr_line (start 128.203999 87.213509) (end 128.240212 88.979223) (layer Edge.Cuts) (width 0.1))
 (gr_line (start 141.54416 112.260754) (end 143.428753 112.260754) (layer Edge.Cuts) (width 0.1))
 (gr_line (start 141.54416 112.907513) (end 141.54416 112.260754) (layer Edge.Cuts) (width 0.1))
 (gr_line (start 134.304176 88.58249) (end 132.81203 87.16315) (layer Edge.Cuts) (width 0.1))
 (gr_line (start 153.035227 123.425301) (end 151.455877 122.587889) (layer Edge.Cuts) (width 0.1))
 (gr_line (start 132.81203 87.16315) (end 131.466303 86.308623) (layer Edge.Cuts) (width 0.1))
 (gr_line (start 143.839383 121.252293) (end 142.659018 119.819034) (layer Edge.Cuts) (width 0.1))
 (gr_line (start 129.548169 101.569282) (end 127.167264 102.676362) (layer Edge.Cuts) (width 0.1))
 (gr_line (start 135.683324 90.980587) (end 134.974633 89.550064) (layer Edge.Cuts) (width 0.1))
 (gr_line (start 146.815176 110.950485) (end 149.238911 108.65994) (layer Edge.Cuts) (width 0.1))
 (gr_line (start 108.480011 132.795455) (end 129.872228 132.95705) (layer Edge.Cuts) (width 0.1))
 (gr_line (start 113.276627 110.725379) (end 110.004567 114.106577) (layer Edge.Cuts) (width 0.1))
 (gr_line (start 145.334943 111.791596) (end 146.815176 110.950485) (layer Edge.Cuts) (width 0.1))
 (gr_line (start 122.60853 108.074626) (end 121.640126 108.135061) (layer Edge.Cuts) (width 0.1))
 (gr_line (start 128.388367 91.160212) (end 128.76 93.46) (layer Edge.Cuts) (width 0.1))
 (gr_line (start 141.225593 118.696991) (end 141.54416 112.907513) (layer Edge.Cuts) (width 0.1))
 (gr_line (start 142.659018 119.819034) (end 141.225593 118.696991) (layer Edge.Cuts) (width 0.1))
 (gr_line (start 135.508649 132.763173) (end 154.43571 132.5325) (layer Edge.Cuts) (width 0.1))
 (gr_line (start 144.482374 122.443642) (end 143.839383 121.252293) (layer Edge.Cuts) (width 0.1))
 (gr_line (start 151.455877 122.587889) (end 144.482374 122.443642) (layer Edge.Cuts) (width 0.1))
 (gr_line (start 154.021633 124.700804) (end 153.035227 123.425301) (layer Edge.Cuts) (width 0.1))
 (gr_line (start 154.43571 126.479059) (end 154.021633 124.700804) (layer Edge.Cuts) (width 0.1))
 (gr_line (start 130.198359 85.635687) (end 129.358953 85.494479) (layer Edge.Cuts) (width 0.1))
 (gr_line (start 129.468258 95.062601) (end 129.509801 98.445187) (layer Edge.Cuts) (width 0.1))
 (gr_line (start 154.43571 132.5325) (end 154.43571 126.479059) (layer Edge.Cuts) (width 0.1))
 (gr_line (start 129.872228 132.95705) (end 129.872228 132.95705) (layer Edge.Cuts) (width 0.1))
 (gr_line (start 134.974633 89.550064) (end 134.304176 88.58249) (layer Edge.Cuts) (width 0.1))
 (gr_line (start 128.76 93.46) (end 129.468258 95.062601) (layer Edge.Cuts) (width 0.1))
 (segment (start 138.5 121.08) (end 139.642999 122.222999) (width 0.25) (layer B.Cu) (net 1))
 (segment (start 139.642999 122.222999) (end 140.332999 122.222999) (width 0.25) (layer B.Cu) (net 1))
 (segment (start 140.332999 122.222999) (end 146.903501 128.793501) (width 0.25) (layer B.Cu) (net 1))
 (segment (start 138.5 119.89) (end 138.5 121.08) (width 0.25) (layer B.Cu) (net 1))
 (segment (start 138.5 119.89) (end 138.741554 119.89) (width 0.25) (layer B.Cu) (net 1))
 (segment (start 138.741554 119.89) (end 138.5 119.648446) (width 0.25) (layer B.Cu) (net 1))
 (segment (start 138.5 119.648446) (end 138.5 118.032) (width 0.25) (layer B.Cu) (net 1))
 (segment (start 117.672 118.032) (end 117.672 116.415554) (width 0.25) (layer B.Cu) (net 1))
 (segment (start 117.672 116.415554) (end 123.746555 110.340999) (width 0.25) (layer B.Cu) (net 1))
 (segment (start 138.5 116.415554) (end 138.5 118.032) (width 0.25) (layer B.Cu) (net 1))
 (segment (start 123.746555 110.340999) (end 132.425445 110.340999) (width 0.25) (layer B.Cu) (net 1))
 (segment (start 132.425445 110.340999) (end 138.5 116.415554) (width 0.25) (layer B.Cu) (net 1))
 (segment (start 117.672 118.032) (end 117.672 119.648446) (width 0.25) (layer B.Cu) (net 1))
 (segment (start 117.672 119.648446) (end 117.672 121.08) (width 0.25) (layer B.Cu) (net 1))
 (segment (start 147.303501 129.029911) (end 147.303501 128.226499) (width 0.25) (layer B.Cu) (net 1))
 (segment (start 148.383501 128.758719) (end 147.851281 128.226499) (width 0.25) (layer B.Cu) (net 1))
 (segment (start 147.303501 128.226499) (end 147.42999 129.1564) (width 0.25) (layer B.Cu) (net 1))
 (segment (start 141.34 131.93) (end 146.194782 131.93) (width 0.25) (layer B.Cu) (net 1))
 (segment (start 146.194782 131.93) (end 148.383501 129.741281) (width 0.25) (layer B.Cu) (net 1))
 (segment (start 148.383501 129.741281) (end 148.383501 128.758719) (width 0.25) (layer B.Cu) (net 1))
 (segment (start 147.851281 128.226499) (end 147.303501 128.226499) (width 0.25) (layer B.Cu) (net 1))
 (segment (start 137.855999 128.445999) (end 141.34 131.93) (width 0.25) (layer B.Cu) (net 1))
 (segment (start 136.975999 128.445999) (end 137.855999 128.445999) (width 0.25) (layer B.Cu) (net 1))
 (segment (start 119.89 129.59) (end 119.89 129.43) (width 0.25) (layer B.Cu) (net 2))
 (segment (start 119.89 129.43) (end 119.89 127.752) (width 0.25) (layer B.Cu) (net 2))
 (segment (start 110.27 130.07) (end 111.069999 129.270001) (width 0.25) (layer B.Cu) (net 2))
 (segment (start 111.069999 129.270001) (end 119.730001 129.270001) (width 0.25) (layer B.Cu) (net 2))
 (segment (start 119.730001 129.270001) (end 119.89 129.43) (width 0.25) (layer B.Cu) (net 2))
 (segment (start 128.086 119.556) (end 136.975999 128.445999) (width 0.25) (layer B.Cu) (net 2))
 (segment (start 119.89 127.752) (end 128.086 119.556) (width 0.25) (layer B.Cu) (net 2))
 (segment (start 134.82 101.8) (end 133.67 101.8) (width 0.25) (layer B.Cu) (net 3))
 (segment (start 133.67 101.8) (end 126.67 108.8) (width 0.25) (layer B.Cu) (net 3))
 (segment (start 121.38 108.8) (end 110.27 119.91) (width 0.25) (layer B.Cu) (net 3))
 (segment (start 126.67 108.8) (end 121.38 108.8) (width 0.25) (layer B.Cu) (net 3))
 (segment (start 147.99 102.04) (end 135.06 102.04) (width 0.25) (layer B.Cu) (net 3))
 (segment (start 135.06 102.04) (end 134.82 101.8) (width 0.25) (layer B.Cu) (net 3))
 (segment (start 140.52 121.61) (end 142.26 121.61) (width 0.25) (layer B.Cu) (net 4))
 (segment (start 142.26 121.61) (end 149.9 129.25) (width 0.25) (layer B.Cu) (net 4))
 (segment (start 147.99 104.58) (end 140.52 112.05) (width 0.25) (layer B.Cu) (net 4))
 (segment (start 140.52 112.05) (end 140.52 121.61) (width 0.25) (layer B.Cu) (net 4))
 (segment (start 134.82 104.34) (end 147.75 104.34) (width 0.25) (layer B.Cu) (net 4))
 (segment (start 147.75 104.34) (end 147.99 104.58) (width 0.25) (layer B.Cu) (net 4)))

